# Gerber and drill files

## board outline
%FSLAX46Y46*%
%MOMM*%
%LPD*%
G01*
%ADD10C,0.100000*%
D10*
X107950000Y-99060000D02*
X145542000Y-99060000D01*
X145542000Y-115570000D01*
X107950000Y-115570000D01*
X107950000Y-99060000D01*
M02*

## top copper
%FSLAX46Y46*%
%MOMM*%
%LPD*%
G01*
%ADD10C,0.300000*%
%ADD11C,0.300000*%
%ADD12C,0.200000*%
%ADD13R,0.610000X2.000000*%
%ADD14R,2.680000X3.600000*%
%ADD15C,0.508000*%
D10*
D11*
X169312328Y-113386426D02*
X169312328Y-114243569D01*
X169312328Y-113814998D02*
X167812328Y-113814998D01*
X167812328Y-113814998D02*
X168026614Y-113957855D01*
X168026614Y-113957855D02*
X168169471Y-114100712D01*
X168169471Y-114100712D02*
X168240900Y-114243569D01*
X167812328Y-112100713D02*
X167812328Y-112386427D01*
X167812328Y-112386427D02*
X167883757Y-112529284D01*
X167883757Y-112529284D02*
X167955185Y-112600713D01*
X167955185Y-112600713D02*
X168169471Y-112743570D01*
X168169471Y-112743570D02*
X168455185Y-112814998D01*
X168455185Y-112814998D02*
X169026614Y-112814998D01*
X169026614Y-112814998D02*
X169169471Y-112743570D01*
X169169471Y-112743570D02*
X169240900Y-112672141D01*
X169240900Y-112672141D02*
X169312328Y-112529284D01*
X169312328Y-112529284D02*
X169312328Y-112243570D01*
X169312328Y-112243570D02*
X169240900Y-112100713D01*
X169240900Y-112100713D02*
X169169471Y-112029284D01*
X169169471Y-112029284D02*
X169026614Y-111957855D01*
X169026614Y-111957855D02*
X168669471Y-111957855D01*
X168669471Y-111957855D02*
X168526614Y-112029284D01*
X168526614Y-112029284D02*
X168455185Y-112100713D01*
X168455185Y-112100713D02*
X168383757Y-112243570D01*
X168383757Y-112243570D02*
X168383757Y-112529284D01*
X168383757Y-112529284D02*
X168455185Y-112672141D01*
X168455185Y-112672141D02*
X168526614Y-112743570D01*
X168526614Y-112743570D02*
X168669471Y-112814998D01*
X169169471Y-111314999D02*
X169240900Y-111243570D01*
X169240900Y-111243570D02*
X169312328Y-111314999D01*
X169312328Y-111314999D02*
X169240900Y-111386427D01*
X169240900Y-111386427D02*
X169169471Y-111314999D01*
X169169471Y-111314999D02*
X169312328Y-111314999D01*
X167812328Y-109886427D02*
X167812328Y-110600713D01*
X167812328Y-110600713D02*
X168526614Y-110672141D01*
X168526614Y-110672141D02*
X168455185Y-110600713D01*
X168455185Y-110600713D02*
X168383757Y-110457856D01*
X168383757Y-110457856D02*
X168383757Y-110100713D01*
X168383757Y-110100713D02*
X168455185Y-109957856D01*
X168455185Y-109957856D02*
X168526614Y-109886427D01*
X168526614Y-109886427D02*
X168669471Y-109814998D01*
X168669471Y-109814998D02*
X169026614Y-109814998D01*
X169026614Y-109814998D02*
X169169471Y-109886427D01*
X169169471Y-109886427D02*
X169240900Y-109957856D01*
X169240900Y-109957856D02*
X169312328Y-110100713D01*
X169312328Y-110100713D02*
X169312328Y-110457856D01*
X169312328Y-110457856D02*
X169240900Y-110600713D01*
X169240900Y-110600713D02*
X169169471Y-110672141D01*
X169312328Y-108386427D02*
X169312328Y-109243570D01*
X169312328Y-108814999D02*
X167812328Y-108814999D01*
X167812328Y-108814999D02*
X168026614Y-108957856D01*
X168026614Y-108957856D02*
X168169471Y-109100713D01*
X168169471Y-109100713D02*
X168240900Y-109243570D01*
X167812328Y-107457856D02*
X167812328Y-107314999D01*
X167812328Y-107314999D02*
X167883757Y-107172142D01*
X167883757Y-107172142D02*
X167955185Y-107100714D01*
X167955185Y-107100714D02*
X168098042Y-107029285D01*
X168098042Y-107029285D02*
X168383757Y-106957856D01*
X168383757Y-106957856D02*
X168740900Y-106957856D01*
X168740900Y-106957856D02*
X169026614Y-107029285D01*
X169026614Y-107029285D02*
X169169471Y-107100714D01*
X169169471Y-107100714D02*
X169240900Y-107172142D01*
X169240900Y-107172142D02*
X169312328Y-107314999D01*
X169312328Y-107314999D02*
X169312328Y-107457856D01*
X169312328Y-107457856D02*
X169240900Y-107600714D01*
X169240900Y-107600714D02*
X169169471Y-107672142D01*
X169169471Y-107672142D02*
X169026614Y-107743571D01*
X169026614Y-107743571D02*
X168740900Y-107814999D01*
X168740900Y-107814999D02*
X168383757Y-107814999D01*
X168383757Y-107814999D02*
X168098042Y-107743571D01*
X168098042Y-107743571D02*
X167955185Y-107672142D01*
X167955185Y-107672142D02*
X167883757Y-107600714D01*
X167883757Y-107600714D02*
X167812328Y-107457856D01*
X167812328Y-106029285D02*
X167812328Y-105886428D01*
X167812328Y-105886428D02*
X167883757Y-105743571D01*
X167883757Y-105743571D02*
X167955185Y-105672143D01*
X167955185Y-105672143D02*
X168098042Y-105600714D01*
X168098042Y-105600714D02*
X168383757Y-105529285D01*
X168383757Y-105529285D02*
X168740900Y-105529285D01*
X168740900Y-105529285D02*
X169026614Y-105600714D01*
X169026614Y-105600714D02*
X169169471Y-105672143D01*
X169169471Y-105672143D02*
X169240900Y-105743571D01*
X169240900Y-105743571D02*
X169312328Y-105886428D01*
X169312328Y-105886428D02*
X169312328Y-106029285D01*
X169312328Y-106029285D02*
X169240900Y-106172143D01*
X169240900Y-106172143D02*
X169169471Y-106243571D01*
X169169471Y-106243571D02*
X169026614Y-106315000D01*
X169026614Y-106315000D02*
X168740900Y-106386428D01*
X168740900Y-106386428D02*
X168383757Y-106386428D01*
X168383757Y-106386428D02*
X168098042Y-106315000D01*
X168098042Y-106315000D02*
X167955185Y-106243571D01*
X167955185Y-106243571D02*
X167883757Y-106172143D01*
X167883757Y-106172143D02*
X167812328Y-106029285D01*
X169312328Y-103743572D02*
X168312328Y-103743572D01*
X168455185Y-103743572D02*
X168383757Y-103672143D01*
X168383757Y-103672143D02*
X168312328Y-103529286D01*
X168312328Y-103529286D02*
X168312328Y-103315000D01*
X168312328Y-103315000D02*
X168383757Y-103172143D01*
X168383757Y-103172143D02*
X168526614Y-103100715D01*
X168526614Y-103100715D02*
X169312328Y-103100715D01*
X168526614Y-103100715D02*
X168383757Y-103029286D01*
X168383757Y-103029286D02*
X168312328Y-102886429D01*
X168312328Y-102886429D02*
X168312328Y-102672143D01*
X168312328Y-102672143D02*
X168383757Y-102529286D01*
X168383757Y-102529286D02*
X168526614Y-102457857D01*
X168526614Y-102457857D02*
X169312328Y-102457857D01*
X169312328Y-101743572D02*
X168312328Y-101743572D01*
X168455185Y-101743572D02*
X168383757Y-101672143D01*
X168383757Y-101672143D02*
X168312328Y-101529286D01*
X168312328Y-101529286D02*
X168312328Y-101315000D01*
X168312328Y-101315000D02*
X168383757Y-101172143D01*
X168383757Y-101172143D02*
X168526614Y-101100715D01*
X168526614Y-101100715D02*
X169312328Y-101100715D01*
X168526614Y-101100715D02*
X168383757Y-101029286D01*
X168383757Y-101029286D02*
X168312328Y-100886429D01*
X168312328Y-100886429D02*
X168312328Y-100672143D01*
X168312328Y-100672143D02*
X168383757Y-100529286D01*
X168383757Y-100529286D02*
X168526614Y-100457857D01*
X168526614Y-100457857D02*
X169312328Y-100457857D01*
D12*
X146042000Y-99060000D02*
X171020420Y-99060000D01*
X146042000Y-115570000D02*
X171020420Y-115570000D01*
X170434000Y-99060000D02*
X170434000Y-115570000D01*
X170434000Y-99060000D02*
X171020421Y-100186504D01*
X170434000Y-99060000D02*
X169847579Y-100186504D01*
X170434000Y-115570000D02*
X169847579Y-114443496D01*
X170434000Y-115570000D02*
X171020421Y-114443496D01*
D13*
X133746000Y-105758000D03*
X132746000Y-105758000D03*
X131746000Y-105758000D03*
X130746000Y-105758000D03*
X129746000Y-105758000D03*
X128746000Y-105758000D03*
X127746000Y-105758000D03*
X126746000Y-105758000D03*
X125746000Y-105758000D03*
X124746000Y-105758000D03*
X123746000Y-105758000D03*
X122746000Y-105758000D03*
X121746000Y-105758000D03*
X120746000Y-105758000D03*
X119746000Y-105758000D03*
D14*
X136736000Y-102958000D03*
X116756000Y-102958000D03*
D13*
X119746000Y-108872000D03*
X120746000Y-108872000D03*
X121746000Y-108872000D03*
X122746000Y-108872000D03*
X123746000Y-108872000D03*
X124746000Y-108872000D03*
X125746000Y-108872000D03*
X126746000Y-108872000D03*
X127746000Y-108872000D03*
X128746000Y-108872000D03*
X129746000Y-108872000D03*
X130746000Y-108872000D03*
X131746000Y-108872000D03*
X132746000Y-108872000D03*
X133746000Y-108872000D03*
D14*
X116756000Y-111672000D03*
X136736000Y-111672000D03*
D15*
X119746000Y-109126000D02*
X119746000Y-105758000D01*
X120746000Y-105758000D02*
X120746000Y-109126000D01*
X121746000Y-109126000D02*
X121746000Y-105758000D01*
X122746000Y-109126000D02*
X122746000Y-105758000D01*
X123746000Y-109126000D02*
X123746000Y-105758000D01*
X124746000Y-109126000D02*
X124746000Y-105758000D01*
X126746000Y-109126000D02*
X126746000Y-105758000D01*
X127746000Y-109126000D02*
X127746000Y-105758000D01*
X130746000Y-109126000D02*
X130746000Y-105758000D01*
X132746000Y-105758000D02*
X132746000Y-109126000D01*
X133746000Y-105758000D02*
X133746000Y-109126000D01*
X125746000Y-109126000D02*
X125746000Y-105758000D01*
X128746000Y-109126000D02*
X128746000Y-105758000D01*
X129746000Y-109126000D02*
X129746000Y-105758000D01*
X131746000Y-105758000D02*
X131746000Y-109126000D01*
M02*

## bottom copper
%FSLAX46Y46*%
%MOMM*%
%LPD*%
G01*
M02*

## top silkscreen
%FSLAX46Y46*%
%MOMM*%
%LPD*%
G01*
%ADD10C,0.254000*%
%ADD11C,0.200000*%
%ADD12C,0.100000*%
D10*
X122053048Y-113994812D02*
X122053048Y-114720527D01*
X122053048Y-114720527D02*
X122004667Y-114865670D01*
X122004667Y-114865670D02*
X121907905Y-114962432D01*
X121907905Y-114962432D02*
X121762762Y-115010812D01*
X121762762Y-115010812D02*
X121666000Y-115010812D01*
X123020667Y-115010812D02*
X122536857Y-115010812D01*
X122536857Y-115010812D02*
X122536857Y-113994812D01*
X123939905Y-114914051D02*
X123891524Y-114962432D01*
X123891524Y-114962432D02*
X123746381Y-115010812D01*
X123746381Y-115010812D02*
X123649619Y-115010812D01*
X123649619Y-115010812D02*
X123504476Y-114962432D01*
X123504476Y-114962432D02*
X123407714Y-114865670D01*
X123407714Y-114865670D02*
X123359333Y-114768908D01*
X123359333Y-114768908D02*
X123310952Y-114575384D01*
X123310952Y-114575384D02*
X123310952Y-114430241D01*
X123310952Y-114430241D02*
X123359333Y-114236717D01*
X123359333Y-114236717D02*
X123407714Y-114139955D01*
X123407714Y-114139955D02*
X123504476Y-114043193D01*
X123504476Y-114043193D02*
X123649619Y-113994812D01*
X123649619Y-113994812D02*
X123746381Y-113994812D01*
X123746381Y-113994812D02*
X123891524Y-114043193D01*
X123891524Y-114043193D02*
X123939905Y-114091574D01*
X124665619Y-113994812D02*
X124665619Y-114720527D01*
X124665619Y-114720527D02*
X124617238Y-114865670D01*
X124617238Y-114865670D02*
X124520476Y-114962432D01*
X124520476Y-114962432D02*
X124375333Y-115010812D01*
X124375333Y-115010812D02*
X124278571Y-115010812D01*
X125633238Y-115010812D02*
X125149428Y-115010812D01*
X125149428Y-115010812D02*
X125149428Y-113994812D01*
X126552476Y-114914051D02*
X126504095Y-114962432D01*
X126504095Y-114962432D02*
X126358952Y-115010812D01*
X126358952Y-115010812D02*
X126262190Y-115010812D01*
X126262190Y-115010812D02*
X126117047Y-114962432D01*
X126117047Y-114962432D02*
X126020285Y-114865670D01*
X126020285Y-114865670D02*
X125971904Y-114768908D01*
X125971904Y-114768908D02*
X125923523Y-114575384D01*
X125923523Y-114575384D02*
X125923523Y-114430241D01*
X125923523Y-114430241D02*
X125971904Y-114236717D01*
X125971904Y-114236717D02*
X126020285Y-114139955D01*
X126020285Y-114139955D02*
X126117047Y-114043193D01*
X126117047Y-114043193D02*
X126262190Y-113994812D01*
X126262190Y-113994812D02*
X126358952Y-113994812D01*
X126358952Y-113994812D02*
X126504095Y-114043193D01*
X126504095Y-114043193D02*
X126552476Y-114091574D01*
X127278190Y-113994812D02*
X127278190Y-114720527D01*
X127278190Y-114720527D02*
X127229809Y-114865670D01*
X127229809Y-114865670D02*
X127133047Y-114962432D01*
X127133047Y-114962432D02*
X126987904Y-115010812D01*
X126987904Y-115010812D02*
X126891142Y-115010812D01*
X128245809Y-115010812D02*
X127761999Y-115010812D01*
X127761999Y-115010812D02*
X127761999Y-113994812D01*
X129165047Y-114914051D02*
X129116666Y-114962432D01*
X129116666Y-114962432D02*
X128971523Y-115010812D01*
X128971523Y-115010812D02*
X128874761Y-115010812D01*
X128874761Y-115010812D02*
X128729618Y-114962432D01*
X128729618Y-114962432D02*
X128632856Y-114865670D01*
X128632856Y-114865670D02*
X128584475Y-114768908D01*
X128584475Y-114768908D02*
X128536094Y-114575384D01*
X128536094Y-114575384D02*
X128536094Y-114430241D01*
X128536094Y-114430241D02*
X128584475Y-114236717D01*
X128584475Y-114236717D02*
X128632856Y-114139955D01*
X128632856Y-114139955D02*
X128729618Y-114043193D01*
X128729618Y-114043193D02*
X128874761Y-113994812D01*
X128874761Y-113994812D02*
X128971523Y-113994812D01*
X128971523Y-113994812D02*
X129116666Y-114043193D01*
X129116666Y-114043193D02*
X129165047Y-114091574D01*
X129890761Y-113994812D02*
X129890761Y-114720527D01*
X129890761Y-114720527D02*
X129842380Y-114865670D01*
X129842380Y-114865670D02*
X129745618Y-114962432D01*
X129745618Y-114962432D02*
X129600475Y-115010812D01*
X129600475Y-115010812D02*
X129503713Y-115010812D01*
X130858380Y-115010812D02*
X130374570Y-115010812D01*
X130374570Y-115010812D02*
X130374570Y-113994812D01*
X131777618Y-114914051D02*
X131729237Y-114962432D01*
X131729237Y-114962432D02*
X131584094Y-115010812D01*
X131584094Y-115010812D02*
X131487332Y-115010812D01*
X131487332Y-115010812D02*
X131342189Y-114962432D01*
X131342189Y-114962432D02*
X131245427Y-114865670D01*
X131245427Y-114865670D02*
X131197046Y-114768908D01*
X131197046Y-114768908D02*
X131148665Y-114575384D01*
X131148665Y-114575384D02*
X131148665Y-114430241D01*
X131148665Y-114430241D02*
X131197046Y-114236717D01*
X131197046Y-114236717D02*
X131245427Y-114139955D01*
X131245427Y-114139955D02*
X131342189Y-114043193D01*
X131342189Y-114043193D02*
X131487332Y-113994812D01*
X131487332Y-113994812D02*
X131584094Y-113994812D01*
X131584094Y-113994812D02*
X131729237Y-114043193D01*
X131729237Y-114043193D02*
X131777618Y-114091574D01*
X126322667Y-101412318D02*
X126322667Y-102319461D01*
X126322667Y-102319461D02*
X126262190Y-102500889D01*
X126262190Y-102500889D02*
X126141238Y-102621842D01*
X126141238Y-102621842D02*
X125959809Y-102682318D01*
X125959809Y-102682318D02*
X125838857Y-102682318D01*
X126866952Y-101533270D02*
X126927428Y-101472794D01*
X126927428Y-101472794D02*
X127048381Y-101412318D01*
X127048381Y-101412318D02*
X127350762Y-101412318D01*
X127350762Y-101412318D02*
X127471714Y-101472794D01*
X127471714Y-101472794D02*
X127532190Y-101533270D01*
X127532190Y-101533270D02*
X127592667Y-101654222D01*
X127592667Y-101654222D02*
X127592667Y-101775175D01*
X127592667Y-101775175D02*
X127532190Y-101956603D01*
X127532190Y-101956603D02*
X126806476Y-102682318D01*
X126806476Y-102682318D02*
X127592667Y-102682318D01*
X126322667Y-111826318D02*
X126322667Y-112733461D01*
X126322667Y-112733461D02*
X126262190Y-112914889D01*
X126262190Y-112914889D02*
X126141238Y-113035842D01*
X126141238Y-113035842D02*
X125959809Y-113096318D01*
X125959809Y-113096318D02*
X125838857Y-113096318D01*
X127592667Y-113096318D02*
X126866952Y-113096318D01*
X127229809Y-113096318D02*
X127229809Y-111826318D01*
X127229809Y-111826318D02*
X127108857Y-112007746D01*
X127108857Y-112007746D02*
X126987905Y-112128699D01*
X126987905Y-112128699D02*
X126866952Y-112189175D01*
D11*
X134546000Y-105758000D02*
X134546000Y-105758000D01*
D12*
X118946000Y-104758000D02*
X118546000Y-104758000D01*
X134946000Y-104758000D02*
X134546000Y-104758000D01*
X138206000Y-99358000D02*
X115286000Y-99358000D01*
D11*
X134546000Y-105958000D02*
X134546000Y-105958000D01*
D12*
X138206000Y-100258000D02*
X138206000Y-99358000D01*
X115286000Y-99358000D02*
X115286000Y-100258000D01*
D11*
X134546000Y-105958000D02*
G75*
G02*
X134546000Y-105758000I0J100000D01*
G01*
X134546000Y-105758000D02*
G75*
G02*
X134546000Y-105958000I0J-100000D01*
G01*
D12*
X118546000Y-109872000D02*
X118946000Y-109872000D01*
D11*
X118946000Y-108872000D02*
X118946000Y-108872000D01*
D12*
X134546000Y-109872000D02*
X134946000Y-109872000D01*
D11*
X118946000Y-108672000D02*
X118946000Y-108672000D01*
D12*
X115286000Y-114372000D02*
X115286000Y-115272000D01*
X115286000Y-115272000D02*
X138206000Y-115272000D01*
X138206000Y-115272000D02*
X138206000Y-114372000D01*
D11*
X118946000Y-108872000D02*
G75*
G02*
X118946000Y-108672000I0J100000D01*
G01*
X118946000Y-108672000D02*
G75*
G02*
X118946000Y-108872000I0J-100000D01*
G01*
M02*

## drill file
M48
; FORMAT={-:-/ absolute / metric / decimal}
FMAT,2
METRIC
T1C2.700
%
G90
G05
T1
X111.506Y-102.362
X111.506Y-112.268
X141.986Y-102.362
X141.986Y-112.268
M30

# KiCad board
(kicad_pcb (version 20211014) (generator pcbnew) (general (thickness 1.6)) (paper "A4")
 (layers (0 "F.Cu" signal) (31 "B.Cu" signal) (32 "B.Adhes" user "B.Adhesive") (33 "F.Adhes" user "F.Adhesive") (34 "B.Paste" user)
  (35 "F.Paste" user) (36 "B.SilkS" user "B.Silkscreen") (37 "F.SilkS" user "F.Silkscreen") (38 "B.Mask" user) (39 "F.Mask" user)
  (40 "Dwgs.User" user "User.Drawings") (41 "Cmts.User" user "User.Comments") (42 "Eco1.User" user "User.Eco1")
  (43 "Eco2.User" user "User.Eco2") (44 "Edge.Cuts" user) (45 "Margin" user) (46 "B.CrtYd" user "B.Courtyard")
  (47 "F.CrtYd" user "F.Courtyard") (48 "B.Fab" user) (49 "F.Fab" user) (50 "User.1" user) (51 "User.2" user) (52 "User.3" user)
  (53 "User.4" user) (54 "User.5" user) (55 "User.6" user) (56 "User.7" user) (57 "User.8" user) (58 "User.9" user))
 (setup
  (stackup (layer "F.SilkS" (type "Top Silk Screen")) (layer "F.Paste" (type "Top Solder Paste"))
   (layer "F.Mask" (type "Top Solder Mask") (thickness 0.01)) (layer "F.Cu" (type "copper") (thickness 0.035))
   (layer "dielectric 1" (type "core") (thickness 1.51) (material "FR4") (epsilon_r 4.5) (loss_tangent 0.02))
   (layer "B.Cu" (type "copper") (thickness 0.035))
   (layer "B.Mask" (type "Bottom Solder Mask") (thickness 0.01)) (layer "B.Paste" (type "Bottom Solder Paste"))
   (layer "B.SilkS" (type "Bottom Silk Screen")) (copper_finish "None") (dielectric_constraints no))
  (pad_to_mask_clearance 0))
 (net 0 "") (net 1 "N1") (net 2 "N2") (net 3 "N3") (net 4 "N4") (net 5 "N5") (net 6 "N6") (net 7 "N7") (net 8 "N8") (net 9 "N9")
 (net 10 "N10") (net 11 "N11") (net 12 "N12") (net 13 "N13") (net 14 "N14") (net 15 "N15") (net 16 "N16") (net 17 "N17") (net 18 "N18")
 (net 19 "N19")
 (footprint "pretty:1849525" (layer "F.Cu") (at 126.746 102.108 180)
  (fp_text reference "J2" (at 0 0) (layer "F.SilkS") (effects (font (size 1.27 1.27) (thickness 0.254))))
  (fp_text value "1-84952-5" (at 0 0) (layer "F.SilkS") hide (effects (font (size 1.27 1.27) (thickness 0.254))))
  (fp_line (start -7.8 -3.65) (end -7.8 -3.65) (layer "F.SilkS") (width 0.2))
  (fp_line (start 7.8 -2.65) (end 8.2 -2.65) (layer "F.SilkS") (width 0.1))
  (fp_line (start -8.2 -2.65) (end -7.8 -2.65) (layer "F.SilkS") (width 0.1))
  (fp_line (start -11.46 2.75) (end 11.46 2.75) (layer "F.SilkS") (width 0.1))
  (fp_line (start -7.8 -3.85) (end -7.8 -3.85) (layer "F.SilkS") (width 0.2))
  (fp_line (start -11.46 1.85) (end -11.46 2.75) (layer "F.SilkS") (width 0.1))
  (fp_line (start 11.46 2.75) (end 11.46 1.85) (layer "F.SilkS") (width 0.1))
  (fp_arc (start -7.8 -3.85) (mid -7.7 -3.75) (end -7.8 -3.65) (layer "F.SilkS") (width 0.2))
  (fp_arc (start -7.8 -3.65) (mid -7.9 -3.75) (end -7.8 -3.85) (layer "F.SilkS") (width 0.2))
  (pad "1" smd rect locked (at -7 -3.65 180) (size 0.61 2) (layers "F.Cu" "F.Paste" "F.Mask") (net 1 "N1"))
  (pad "2" smd rect locked (at -6 -3.65 180) (size 0.61 2) (layers "F.Cu" "F.Paste" "F.Mask") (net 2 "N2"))
  (pad "3" smd rect locked (at -5 -3.65 180) (size 0.61 2) (layers "F.Cu" "F.Paste" "F.Mask") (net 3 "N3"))
  (pad "4" smd rect locked (at -4 -3.65 180) (size 0.61 2) (layers "F.Cu" "F.Paste" "F.Mask") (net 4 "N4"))
  (pad "5" smd rect locked (at -3 -3.65 180) (size 0.61 2) (layers "F.Cu" "F.Paste" "F.Mask") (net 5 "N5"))
  (pad "6" smd rect locked (at -2 -3.65 180) (size 0.61 2) (layers "F.Cu" "F.Paste" "F.Mask") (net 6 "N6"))
  (pad "7" smd rect locked (at -1 -3.65 180) (size 0.61 2) (layers "F.Cu" "F.Paste" "F.Mask") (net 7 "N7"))
  (pad "8" smd rect locked (at 0 -3.65 180) (size 0.61 2) (layers "F.Cu" "F.Paste" "F.Mask") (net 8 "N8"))
  (pad "9" smd rect locked (at 1 -3.65 180) (size 0.61 2) (layers "F.Cu" "F.Paste" "F.Mask") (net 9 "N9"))
  (pad "10" smd rect locked (at 2 -3.65 180) (size 0.61 2) (layers "F.Cu" "F.Paste" "F.Mask") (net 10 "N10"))
  (pad "11" smd rect locked (at 3 -3.65 180) (size 0.61 2) (layers "F.Cu" "F.Paste" "F.Mask") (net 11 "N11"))
  (pad "12" smd rect locked (at 4 -3.65 180) (size 0.61 2) (layers "F.Cu" "F.Paste" "F.Mask") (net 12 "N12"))
  (pad "13" smd rect locked (at 5 -3.65 180) (size 0.61 2) (layers "F.Cu" "F.Paste" "F.Mask") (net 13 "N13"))
  (pad "14" smd rect locked (at 6 -3.65 180) (size 0.61 2) (layers "F.Cu" "F.Paste" "F.Mask") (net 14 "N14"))
  (pad "15" smd rect locked (at 7 -3.65 180) (size 0.61 2) (layers "F.Cu" "F.Paste" "F.Mask") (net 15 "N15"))
  (pad "MP1" smd rect locked (at -9.99 -0.85 180) (size 2.68 3.6) (layers "F.Cu" "F.Paste" "F.Mask") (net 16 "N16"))
  (pad "MP2" smd rect locked (at 9.99 -0.85 180) (size 2.68 3.6) (layers "F.Cu" "F.Paste" "F.Mask") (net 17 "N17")))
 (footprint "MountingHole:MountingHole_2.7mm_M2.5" (layer "F.Cu") (at 141.986 102.362)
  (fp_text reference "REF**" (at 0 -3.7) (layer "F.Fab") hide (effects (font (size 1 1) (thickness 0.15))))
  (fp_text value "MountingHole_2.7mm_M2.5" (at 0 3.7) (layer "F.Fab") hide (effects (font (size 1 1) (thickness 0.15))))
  (pad "" np_thru_hole circle locked (at 0 0) (size 2.7 2.7) (drill 2.7) (layers *.Cu *.Mask)))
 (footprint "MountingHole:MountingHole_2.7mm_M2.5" (layer "F.Cu") (at 141.986 112.268)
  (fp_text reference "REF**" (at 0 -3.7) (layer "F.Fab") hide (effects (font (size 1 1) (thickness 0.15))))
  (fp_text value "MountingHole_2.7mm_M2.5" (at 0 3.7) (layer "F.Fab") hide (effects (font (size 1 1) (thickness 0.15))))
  (pad "" np_thru_hole circle locked (at 0 0) (size 2.7 2.7) (drill 2.7) (layers *.Cu *.Mask)))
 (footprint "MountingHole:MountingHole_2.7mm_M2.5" (layer "F.Cu") (at 111.506 102.362)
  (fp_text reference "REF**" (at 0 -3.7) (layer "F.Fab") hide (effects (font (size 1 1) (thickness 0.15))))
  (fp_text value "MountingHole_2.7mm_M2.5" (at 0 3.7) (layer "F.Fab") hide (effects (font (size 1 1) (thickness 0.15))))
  (pad "" np_thru_hole circle locked (at 0 0) (size 2.7 2.7) (drill 2.7) (layers *.Cu *.Mask)))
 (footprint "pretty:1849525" (layer "F.Cu") (at 126.746 112.522)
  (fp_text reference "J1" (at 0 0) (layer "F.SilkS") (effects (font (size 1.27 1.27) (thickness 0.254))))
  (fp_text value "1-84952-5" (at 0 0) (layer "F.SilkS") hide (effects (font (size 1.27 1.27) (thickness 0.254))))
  (fp_line (start -8.2 -2.65) (end -7.8 -2.65) (layer "F.SilkS") (width 0.1))
  (fp_line (start -7.8 -3.65) (end -7.8 -3.65) (layer "F.SilkS") (width 0.2))
  (fp_line (start 7.8 -2.65) (end 8.2 -2.65) (layer "F.SilkS") (width 0.1))
  (fp_line (start -7.8 -3.85) (end -7.8 -3.85) (layer "F.SilkS") (width 0.2))
  (fp_line (start -11.46 1.85) (end -11.46 2.75) (layer "F.SilkS") (width 0.1))
  (fp_line (start -11.46 2.75) (end 11.46 2.75) (layer "F.SilkS") (width 0.1))
  (fp_line (start 11.46 2.75) (end 11.46 1.85) (layer "F.SilkS") (width 0.1))
  (fp_arc (start -7.8 -3.65) (mid -7.9 -3.75) (end -7.8 -3.85) (layer "F.SilkS") (width 0.2))
  (fp_arc (start -7.8 -3.85) (mid -7.7 -3.75) (end -7.8 -3.65) (layer "F.SilkS") (width 0.2))
  (pad "1" smd rect locked (at -7 -3.65) (size 0.61 2) (layers "F.Cu" "F.Paste" "F.Mask") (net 15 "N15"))
  (pad "2" smd rect locked (at -6 -3.65) (size 0.61 2) (layers "F.Cu" "F.Paste" "F.Mask") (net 14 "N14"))
  (pad "3" smd rect locked (at -5 -3.65) (size 0.61 2) (layers "F.Cu" "F.Paste" "F.Mask") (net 13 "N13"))
  (pad "4" smd rect locked (at -4 -3.65) (size 0.61 2) (layers "F.Cu" "F.Paste" "F.Mask") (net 12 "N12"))
  (pad "5" smd rect locked (at -3 -3.65) (size 0.61 2) (layers "F.Cu" "F.Paste" "F.Mask") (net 11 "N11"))
  (pad "6" smd rect locked (at -2 -3.65) (size 0.61 2) (layers "F.Cu" "F.Paste" "F.Mask") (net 10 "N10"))
  (pad "7" smd rect locked (at -1 -3.65) (size 0.61 2) (layers "F.Cu" "F.Paste" "F.Mask") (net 9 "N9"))
  (pad "8" smd rect locked (at 0 -3.65) (size 0.61 2) (layers "F.Cu" "F.Paste" "F.Mask") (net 8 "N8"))
  (pad "9" smd rect locked (at 1 -3.65) (size 0.61 2) (layers "F.Cu" "F.Paste" "F.Mask") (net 7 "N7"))
  (pad "10" smd rect locked (at 2 -3.65) (size 0.61 2) (layers "F.Cu" "F.Paste" "F.Mask") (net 6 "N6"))
  (pad "11" smd rect locked (at 3 -3.65) (size 0.61 2) (layers "F.Cu" "F.Paste" "F.Mask") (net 5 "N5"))
  (pad "12" smd rect locked (at 4 -3.65) (size 0.61 2) (layers "F.Cu" "F.Paste" "F.Mask") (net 4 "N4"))
  (pad "13" smd rect locked (at 5 -3.65) (size 0.61 2) (layers "F.Cu" "F.Paste" "F.Mask") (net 3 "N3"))
  (pad "14" smd rect locked (at 6 -3.65) (size 0.61 2) (layers "F.Cu" "F.Paste" "F.Mask") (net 2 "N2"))
  (pad "15" smd rect locked (at 7 -3.65) (size 0.61 2) (layers "F.Cu" "F.Paste" "F.Mask") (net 1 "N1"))
  (pad "MP1" smd rect locked (at -9.99 -0.85) (size 2.68 3.6) (layers "F.Cu" "F.Paste" "F.Mask") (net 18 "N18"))
  (pad "MP2" smd rect locked (at 9.99 -0.85) (size 2.68 3.6) (layers "F.Cu" "F.Paste" "F.Mask") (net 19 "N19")))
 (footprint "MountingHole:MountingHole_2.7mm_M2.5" (layer "F.Cu") (at 111.506 112.268)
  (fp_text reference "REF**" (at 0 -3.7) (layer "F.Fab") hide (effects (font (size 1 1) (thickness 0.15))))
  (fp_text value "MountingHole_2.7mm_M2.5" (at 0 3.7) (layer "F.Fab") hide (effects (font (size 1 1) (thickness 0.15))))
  (pad "" np_thru_hole circle locked (at 0 0) (size 2.7 2.7) (drill 2.7) (layers *.Cu *.Mask)))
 (gr_rect (start 145.542 99.06) (end 107.95 115.57) (layer "Edge.Cuts") (width 0.1) (fill none))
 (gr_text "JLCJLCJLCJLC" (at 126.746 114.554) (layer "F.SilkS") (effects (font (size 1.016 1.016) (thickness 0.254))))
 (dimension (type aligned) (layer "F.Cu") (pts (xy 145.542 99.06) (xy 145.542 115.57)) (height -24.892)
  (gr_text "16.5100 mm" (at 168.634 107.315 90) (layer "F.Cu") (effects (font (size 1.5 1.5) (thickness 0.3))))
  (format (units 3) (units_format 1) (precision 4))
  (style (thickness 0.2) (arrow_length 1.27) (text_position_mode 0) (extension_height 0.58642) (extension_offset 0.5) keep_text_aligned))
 (segment (start 119.746 109.126) (end 119.746 105.758) (width 0.508) (layer "F.Cu") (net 15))
 (segment (start 120.746 105.758) (end 120.746 109.126) (width 0.508) (layer "F.Cu") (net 14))
 (segment (start 121.746 109.126) (end 121.746 105.758) (width 0.508) (layer "F.Cu") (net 13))
 (segment (start 122.746 109.126) (end 122.746 105.758) (width 0.508) (layer "F.Cu") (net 12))
 (segment (start 123.746 109.126) (end 123.746 105.758) (width 0.508) (layer "F.Cu") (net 11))
 (segment (start 124.746 109.126) (end 124.746 105.758) (width 0.508) (layer "F.Cu") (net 10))
 (segment (start 126.746 109.126) (end 126.746 105.758) (width 0.508) (layer "F.Cu") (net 8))
 (segment (start 127.746 109.126) (end 127.746 105.758) (width 0.508) (layer "F.Cu") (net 7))
 (segment (start 130.746 109.126) (end 130.746 105.758) (width 0.508) (layer "F.Cu") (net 4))
 (segment (start 132.746 105.758) (end 132.746 109.126) (width 0.508) (layer "F.Cu") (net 2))
 (segment (start 133.746 105.758) (end 133.746 109.126) (width 0.508) (layer "F.Cu") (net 1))
 (segment (start 125.746 109.126) (end 125.746 105.758) (width 0.508) (layer "F.Cu") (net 9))
 (segment (start 128.746 109.126) (end 128.746 105.758) (width 0.508) (layer "F.Cu") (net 6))
 (segment (start 129.746 109.126) (end 129.746 105.758) (width 0.508) (layer "F.Cu") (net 5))
 (segment (start 131.746 105.758) (end 131.746 109.126) (width 0.508) (layer "F.Cu") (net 3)))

